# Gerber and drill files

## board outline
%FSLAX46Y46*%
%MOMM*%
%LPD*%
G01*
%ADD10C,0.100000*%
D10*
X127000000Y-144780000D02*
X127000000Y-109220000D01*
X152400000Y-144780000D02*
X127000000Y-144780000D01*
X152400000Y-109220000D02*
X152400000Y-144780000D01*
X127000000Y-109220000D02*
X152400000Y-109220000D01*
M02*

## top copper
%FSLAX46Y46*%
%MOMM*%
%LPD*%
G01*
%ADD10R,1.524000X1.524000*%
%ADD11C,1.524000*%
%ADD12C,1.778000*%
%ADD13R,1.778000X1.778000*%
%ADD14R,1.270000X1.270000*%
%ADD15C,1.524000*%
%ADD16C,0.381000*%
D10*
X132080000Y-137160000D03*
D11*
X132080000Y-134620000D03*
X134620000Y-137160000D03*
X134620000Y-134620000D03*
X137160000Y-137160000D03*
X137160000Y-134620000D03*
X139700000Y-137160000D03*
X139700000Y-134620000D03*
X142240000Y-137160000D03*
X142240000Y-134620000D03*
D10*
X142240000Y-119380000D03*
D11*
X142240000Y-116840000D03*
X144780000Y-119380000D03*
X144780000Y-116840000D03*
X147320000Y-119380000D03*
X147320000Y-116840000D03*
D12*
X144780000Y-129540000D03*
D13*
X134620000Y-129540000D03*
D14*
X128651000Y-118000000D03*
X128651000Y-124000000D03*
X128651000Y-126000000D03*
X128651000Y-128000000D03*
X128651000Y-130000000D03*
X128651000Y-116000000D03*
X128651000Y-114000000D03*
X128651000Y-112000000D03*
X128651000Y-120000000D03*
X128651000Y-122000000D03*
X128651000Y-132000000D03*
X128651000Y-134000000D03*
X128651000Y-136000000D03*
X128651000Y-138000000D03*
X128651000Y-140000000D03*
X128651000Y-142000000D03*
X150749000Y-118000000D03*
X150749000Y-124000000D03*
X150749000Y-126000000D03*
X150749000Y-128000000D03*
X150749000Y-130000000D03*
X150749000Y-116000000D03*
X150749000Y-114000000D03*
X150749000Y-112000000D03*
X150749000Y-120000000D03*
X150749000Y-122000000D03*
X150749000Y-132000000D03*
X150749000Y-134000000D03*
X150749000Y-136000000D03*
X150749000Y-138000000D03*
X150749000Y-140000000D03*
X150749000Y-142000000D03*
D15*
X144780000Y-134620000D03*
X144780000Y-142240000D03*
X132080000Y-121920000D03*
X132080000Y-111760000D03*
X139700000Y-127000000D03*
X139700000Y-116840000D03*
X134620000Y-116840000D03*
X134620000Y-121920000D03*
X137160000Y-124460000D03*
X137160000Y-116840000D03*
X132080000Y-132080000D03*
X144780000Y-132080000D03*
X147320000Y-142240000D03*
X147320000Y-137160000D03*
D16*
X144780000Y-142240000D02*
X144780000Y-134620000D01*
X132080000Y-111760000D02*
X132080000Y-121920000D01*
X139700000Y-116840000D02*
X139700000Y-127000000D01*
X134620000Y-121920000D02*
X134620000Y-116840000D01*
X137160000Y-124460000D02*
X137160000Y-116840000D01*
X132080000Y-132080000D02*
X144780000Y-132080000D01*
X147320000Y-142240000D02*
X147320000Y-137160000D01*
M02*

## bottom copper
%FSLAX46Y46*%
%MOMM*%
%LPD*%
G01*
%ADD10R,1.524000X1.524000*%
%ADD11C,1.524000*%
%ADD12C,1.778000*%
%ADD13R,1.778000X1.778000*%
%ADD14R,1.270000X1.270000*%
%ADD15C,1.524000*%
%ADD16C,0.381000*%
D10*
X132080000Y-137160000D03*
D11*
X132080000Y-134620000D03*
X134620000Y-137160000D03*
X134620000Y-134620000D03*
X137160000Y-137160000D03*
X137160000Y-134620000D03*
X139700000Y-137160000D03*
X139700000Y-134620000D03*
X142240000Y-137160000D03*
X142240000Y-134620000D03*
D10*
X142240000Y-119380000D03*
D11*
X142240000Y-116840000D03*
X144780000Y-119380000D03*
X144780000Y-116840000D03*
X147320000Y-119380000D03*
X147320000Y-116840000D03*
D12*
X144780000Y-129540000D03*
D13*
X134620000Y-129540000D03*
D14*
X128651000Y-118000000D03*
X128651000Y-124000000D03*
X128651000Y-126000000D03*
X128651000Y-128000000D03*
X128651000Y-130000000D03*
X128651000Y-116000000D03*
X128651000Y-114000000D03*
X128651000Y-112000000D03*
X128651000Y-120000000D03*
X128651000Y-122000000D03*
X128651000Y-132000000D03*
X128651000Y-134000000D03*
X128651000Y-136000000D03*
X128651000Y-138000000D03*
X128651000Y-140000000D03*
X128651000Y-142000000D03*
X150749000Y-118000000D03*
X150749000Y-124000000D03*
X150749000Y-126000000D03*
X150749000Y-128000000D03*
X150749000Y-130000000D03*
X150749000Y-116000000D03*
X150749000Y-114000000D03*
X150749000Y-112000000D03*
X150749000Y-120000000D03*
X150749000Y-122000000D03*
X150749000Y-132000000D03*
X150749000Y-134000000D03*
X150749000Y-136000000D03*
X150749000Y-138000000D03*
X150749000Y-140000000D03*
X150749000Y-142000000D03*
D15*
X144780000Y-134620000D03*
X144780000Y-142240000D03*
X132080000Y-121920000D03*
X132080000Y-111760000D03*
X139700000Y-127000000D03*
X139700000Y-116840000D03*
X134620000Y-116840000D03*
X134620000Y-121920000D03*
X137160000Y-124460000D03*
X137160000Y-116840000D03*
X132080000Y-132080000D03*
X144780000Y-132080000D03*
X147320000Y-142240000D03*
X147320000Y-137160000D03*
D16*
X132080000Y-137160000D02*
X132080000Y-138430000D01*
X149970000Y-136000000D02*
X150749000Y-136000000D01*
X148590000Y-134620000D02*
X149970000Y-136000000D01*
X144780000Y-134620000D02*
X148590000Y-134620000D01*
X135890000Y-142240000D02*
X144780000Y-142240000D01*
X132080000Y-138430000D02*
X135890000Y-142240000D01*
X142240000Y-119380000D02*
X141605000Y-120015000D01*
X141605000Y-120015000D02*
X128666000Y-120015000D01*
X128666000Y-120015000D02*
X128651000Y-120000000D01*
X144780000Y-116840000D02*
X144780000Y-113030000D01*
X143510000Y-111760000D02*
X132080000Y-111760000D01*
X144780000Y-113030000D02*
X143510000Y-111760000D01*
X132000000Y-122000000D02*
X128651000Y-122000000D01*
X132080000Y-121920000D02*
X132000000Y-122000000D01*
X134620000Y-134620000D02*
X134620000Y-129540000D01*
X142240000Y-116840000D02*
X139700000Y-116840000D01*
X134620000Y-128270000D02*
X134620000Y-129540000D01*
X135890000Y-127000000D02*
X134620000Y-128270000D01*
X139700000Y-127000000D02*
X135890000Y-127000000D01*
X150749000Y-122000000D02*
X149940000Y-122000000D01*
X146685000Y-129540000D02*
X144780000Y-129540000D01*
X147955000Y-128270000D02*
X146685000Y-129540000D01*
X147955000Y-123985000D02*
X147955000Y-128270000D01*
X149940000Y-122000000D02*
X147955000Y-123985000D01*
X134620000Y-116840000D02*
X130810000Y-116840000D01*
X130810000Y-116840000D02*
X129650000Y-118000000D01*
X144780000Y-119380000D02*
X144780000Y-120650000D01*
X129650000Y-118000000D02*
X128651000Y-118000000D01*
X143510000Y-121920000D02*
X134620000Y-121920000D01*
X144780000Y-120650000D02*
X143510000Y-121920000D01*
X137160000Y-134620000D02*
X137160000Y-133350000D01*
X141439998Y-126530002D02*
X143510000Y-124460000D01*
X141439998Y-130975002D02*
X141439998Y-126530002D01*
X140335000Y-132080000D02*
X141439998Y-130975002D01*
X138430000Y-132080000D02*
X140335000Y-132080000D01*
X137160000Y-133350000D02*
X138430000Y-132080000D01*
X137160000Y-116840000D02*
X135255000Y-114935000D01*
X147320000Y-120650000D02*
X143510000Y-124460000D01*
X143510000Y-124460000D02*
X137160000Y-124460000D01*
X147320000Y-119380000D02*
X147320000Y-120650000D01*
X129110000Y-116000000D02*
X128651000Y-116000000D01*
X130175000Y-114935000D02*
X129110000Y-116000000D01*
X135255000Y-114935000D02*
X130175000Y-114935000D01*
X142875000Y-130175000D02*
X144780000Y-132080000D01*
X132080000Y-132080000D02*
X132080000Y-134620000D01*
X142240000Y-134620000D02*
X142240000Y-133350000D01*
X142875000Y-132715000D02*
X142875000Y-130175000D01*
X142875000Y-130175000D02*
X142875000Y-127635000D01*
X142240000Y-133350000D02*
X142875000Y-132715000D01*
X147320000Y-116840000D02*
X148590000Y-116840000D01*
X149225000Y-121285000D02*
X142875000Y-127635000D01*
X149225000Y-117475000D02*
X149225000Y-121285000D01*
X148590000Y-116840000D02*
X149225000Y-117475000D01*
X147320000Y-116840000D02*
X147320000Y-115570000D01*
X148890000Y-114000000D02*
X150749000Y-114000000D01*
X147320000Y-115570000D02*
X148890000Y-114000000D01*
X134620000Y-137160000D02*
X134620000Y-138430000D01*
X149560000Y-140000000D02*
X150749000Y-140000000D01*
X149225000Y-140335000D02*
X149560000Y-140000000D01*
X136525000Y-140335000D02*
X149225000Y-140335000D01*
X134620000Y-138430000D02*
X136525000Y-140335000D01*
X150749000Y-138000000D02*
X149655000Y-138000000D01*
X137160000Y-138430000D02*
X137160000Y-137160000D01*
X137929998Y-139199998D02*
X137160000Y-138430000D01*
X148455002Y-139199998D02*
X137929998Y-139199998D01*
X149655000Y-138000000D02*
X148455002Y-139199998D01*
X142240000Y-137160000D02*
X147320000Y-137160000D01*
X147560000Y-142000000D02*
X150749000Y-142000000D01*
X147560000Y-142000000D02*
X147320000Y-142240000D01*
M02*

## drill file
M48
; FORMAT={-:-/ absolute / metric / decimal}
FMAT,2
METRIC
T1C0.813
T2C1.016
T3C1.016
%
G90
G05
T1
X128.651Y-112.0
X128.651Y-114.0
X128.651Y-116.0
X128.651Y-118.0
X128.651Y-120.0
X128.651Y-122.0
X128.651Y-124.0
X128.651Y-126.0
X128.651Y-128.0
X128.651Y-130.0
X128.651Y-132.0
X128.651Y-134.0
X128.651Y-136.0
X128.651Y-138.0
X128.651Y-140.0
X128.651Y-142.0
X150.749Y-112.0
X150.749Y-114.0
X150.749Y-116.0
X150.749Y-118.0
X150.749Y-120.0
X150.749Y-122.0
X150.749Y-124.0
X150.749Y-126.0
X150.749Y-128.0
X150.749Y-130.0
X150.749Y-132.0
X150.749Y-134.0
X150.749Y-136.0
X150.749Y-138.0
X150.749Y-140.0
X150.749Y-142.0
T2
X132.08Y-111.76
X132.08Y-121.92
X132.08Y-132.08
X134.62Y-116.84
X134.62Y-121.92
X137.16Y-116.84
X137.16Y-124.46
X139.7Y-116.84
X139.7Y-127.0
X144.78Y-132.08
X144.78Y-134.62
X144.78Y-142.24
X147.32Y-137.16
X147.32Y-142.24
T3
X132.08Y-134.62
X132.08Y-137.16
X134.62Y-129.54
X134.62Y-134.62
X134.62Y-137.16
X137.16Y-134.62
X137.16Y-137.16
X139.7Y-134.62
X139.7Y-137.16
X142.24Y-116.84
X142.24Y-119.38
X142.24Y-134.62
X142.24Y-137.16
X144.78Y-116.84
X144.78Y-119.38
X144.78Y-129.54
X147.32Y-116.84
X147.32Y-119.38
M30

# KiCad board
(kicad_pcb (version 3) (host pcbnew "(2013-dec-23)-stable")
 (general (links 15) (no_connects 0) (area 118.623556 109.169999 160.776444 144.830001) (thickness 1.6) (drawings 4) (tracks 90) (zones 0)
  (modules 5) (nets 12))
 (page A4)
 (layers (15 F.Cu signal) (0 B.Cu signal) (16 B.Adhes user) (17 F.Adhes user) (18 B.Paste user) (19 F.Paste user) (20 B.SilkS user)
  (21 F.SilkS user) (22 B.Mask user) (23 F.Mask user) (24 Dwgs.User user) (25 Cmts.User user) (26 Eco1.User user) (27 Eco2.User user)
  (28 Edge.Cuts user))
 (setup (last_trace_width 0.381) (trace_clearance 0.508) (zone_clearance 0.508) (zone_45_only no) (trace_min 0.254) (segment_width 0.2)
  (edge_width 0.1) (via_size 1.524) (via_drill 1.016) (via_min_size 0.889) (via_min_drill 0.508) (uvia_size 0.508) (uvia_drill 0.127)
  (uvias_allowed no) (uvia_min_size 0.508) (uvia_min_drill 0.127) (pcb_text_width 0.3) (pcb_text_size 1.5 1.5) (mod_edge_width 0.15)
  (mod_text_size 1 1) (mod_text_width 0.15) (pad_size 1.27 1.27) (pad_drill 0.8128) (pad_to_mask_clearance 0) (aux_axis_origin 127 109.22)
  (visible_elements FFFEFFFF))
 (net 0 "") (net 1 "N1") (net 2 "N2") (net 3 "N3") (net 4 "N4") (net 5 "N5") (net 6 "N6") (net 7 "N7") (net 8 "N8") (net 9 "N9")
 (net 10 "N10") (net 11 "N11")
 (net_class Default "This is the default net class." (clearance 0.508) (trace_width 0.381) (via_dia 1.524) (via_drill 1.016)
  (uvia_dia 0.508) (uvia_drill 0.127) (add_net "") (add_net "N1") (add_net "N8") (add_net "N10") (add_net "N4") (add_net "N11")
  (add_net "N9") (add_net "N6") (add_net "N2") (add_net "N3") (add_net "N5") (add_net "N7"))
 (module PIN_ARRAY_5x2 (layer F.Cu) (at 137.16 135.89)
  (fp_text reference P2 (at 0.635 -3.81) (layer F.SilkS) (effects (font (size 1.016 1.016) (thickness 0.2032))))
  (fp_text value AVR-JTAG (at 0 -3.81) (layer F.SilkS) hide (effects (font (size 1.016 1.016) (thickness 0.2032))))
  (pad 1 thru_hole rect (at -5.08 1.27) (size 1.524 1.524) (drill 1.016) (layers *.Cu *.Mask F.SilkS) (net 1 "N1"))
  (pad 2 thru_hole circle (at -5.08 -1.27) (size 1.524 1.524) (drill 1.016) (layers *.Cu *.Mask F.SilkS) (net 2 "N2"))
  (pad 3 thru_hole circle (at -2.54 1.27) (size 1.524 1.524) (drill 1.016) (layers *.Cu *.Mask F.SilkS) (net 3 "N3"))
  (pad 4 thru_hole circle (at -2.54 -1.27) (size 1.524 1.524) (drill 1.016) (layers *.Cu *.Mask F.SilkS) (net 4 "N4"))
  (pad 5 thru_hole circle (at 0 1.27) (size 1.524 1.524) (drill 1.016) (layers *.Cu *.Mask F.SilkS) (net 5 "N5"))
  (pad 6 thru_hole circle (at 0 -1.27) (size 1.524 1.524) (drill 1.016) (layers *.Cu *.Mask F.SilkS) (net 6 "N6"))
  (pad 7 thru_hole circle (at 2.54 1.27) (size 1.524 1.524) (drill 1.016) (layers *.Cu *.Mask F.SilkS))
  (pad 8 thru_hole circle (at 2.54 -1.27) (size 1.524 1.524) (drill 1.016) (layers *.Cu *.Mask F.SilkS))
  (pad 9 thru_hole circle (at 5.08 1.27) (size 1.524 1.524) (drill 1.016) (layers *.Cu *.Mask F.SilkS) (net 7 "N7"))
  (pad 10 thru_hole circle (at 5.08 -1.27) (size 1.524 1.524) (drill 1.016) (layers *.Cu *.Mask F.SilkS) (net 2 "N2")))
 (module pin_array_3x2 (layer F.Cu) (at 144.78 118.11)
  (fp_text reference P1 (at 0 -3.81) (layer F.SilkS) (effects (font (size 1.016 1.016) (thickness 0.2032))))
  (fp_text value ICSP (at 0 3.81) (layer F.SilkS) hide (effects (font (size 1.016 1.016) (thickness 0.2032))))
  (pad 1 thru_hole rect (at -2.54 1.27) (size 1.524 1.524) (drill 1.016) (layers *.Cu *.Mask F.SilkS) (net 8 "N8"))
  (pad 2 thru_hole circle (at -2.54 -1.27) (size 1.524 1.524) (drill 1.016) (layers *.Cu *.Mask F.SilkS) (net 4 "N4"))
  (pad 3 thru_hole circle (at 0 1.27) (size 1.524 1.524) (drill 1.016) (layers *.Cu *.Mask F.SilkS) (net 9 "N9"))
  (pad 4 thru_hole circle (at 0 -1.27) (size 1.524 1.524) (drill 1.016) (layers *.Cu *.Mask F.SilkS) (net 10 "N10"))
  (pad 5 thru_hole circle (at 2.54 1.27) (size 1.524 1.524) (drill 1.016) (layers *.Cu *.Mask F.SilkS) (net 6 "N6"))
  (pad 6 thru_hole circle (at 2.54 -1.27) (size 1.524 1.524) (drill 1.016) (layers *.Cu *.Mask F.SilkS) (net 2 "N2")))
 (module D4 (layer F.Cu) (at 139.7 129.54 180)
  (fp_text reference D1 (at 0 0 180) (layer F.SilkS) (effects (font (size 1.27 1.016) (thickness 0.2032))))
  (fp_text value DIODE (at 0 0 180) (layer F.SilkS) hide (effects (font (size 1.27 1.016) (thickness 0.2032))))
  (pad 1 thru_hole circle (at -5.08 0 180) (size 1.778 1.778) (drill 1.016) (layers *.Cu *.Mask F.SilkS) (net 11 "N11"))
  (pad 2 thru_hole rect (at 5.08 0 180) (size 1.778 1.778) (drill 1.016) (layers *.Cu *.Mask F.SilkS) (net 4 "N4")))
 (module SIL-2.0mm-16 (layer F.Cu) (at 128.651 127)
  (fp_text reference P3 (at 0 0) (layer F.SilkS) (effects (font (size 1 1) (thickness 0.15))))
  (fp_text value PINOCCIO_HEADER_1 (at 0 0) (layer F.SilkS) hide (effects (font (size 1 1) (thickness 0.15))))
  (pad 4 thru_hole rect (at 0 -9) (size 1.27 1.27) (drill 0.8128) (layers *.Cu *.Mask F.SilkS) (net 9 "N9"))
  (pad 7 thru_hole rect (at 0 -3) (size 1.27 1.27) (drill 0.8128) (layers *.Cu *.Mask F.SilkS))
  (pad 8 thru_hole rect (at 0 -1) (size 1.27 1.27) (drill 0.8128) (layers *.Cu *.Mask F.SilkS))
  (pad 9 thru_hole rect (at 0 1) (size 1.27 1.27) (drill 0.8128) (layers *.Cu *.Mask F.SilkS))
  (pad 10 thru_hole rect (at 0 3) (size 1.27 1.27) (drill 0.8128) (layers *.Cu *.Mask F.SilkS))
  (pad 3 thru_hole rect (at 0 -11) (size 1.27 1.27) (drill 0.8128) (layers *.Cu *.Mask F.SilkS) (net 6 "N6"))
  (pad 2 thru_hole rect (at 0 -13) (size 1.27 1.27) (drill 0.8128) (layers *.Cu *.Mask F.SilkS))
  (pad 1 thru_hole rect (at 0 -15) (size 1.27 1.27) (drill 0.8128) (layers *.Cu *.Mask F.SilkS))
  (pad 5 thru_hole rect (at 0 -7) (size 1.27 1.27) (drill 0.8128) (layers *.Cu *.Mask F.SilkS) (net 8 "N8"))
  (pad 6 thru_hole rect (at 0 -5) (size 1.27 1.27) (drill 0.8128) (layers *.Cu *.Mask F.SilkS) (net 10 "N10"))
  (pad 11 thru_hole rect (at 0 5) (size 1.27 1.27) (drill 0.8128) (layers *.Cu *.Mask F.SilkS))
  (pad 12 thru_hole rect (at 0 7) (size 1.27 1.27) (drill 0.8128) (layers *.Cu *.Mask F.SilkS))
  (pad 13 thru_hole rect (at 0 9) (size 1.27 1.27) (drill 0.8128) (layers *.Cu *.Mask F.SilkS))
  (pad 14 thru_hole rect (at 0 11) (size 1.27 1.27) (drill 0.8128) (layers *.Cu *.Mask F.SilkS))
  (pad 15 thru_hole rect (at 0 13) (size 1.27 1.27) (drill 0.8128) (layers *.Cu *.Mask F.SilkS))
  (pad 16 thru_hole rect (at 0 15) (size 1.27 1.27) (drill 0.8128) (layers *.Cu *.Mask F.SilkS)))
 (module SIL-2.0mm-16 (layer F.Cu) (at 150.749 127)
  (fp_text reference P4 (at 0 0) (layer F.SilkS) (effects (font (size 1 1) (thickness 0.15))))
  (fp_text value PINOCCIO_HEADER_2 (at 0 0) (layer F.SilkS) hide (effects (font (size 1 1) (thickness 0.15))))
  (pad 4 thru_hole rect (at 0 -9) (size 1.27 1.27) (drill 0.8128) (layers *.Cu *.Mask F.SilkS))
  (pad 7 thru_hole rect (at 0 -3) (size 1.27 1.27) (drill 0.8128) (layers *.Cu *.Mask F.SilkS))
  (pad 8 thru_hole rect (at 0 -1) (size 1.27 1.27) (drill 0.8128) (layers *.Cu *.Mask F.SilkS))
  (pad 9 thru_hole rect (at 0 1) (size 1.27 1.27) (drill 0.8128) (layers *.Cu *.Mask F.SilkS))
  (pad 10 thru_hole rect (at 0 3) (size 1.27 1.27) (drill 0.8128) (layers *.Cu *.Mask F.SilkS))
  (pad 3 thru_hole rect (at 0 -11) (size 1.27 1.27) (drill 0.8128) (layers *.Cu *.Mask F.SilkS))
  (pad 2 thru_hole rect (at 0 -13) (size 1.27 1.27) (drill 0.8128) (layers *.Cu *.Mask F.SilkS) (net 2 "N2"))
  (pad 1 thru_hole rect (at 0 -15) (size 1.27 1.27) (drill 0.8128) (layers *.Cu *.Mask F.SilkS))
  (pad 5 thru_hole rect (at 0 -7) (size 1.27 1.27) (drill 0.8128) (layers *.Cu *.Mask F.SilkS))
  (pad 6 thru_hole rect (at 0 -5) (size 1.27 1.27) (drill 0.8128) (layers *.Cu *.Mask F.SilkS) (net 11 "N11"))
  (pad 11 thru_hole rect (at 0 5) (size 1.27 1.27) (drill 0.8128) (layers *.Cu *.Mask F.SilkS))
  (pad 12 thru_hole rect (at 0 7) (size 1.27 1.27) (drill 0.8128) (layers *.Cu *.Mask F.SilkS))
  (pad 13 thru_hole rect (at 0 9) (size 1.27 1.27) (drill 0.8128) (layers *.Cu *.Mask F.SilkS) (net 1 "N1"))
  (pad 14 thru_hole rect (at 0 11) (size 1.27 1.27) (drill 0.8128) (layers *.Cu *.Mask F.SilkS) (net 5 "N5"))
  (pad 15 thru_hole rect (at 0 13) (size 1.27 1.27) (drill 0.8128) (layers *.Cu *.Mask F.SilkS) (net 3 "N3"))
  (pad 16 thru_hole rect (at 0 15) (size 1.27 1.27) (drill 0.8128) (layers *.Cu *.Mask F.SilkS) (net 7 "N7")))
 (gr_line (start 127 144.78) (end 127 109.22) (angle 90) (layer Edge.Cuts) (width 0.1))
 (gr_line (start 152.4 144.78) (end 127 144.78) (angle 90) (layer Edge.Cuts) (width 0.1))
 (gr_line (start 152.4 109.22) (end 152.4 144.78) (angle 90) (layer Edge.Cuts) (width 0.1))
 (gr_line (start 127 109.22) (end 152.4 109.22) (angle 90) (layer Edge.Cuts) (width 0.1))
 (segment (start 132.08 137.16) (end 132.08 138.43) (width 0.381) (layer B.Cu) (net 1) (status 10))
 (segment (start 149.97 136) (end 150.749 136) (width 0.381) (layer B.Cu) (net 1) (status 20))
 (segment (start 148.59 134.62) (end 149.97 136) (width 0.381) (layer B.Cu) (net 1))
 (segment (start 144.78 134.62) (end 148.59 134.62) (width 0.381) (layer B.Cu) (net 1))
 (via (at 144.78 134.62) (size 1.524) (layers F.Cu B.Cu) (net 1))
 (segment (start 144.78 142.24) (end 144.78 134.62) (width 0.381) (layer F.Cu) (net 1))
 (via (at 144.78 142.24) (size 1.524) (layers F.Cu B.Cu) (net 1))
 (segment (start 135.89 142.24) (end 144.78 142.24) (width 0.381) (layer B.Cu) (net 1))
 (segment (start 132.08 138.43) (end 135.89 142.24) (width 0.381) (layer B.Cu) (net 1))
 (segment (start 142.24 119.38) (end 141.605 120.015) (width 0.381) (layer B.Cu) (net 8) (status 30))
 (segment (start 141.605 120.015) (end 128.666 120.015) (width 0.381) (layer B.Cu) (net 8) (status 30))
 (segment (start 128.666 120.015) (end 128.651 120) (width 0.381) (layer B.Cu) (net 8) (status 30))
 (segment (start 144.78 116.84) (end 144.78 113.03) (width 0.381) (layer B.Cu) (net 10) (status 10))
 (segment (start 143.51 111.76) (end 132.08 111.76) (width 0.381) (layer B.Cu) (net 10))
 (segment (start 144.78 113.03) (end 143.51 111.76) (width 0.381) (layer B.Cu) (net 10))
 (segment (start 132 122) (end 128.651 122) (width 0.381) (layer B.Cu) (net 10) (status 20))
 (segment (start 132.08 121.92) (end 132 122) (width 0.381) (layer B.Cu) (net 10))
 (via (at 132.08 121.92) (size 1.524) (layers F.Cu B.Cu) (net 10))
 (segment (start 132.08 111.76) (end 132.08 121.92) (width 0.381) (layer F.Cu) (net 10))
 (via (at 132.08 111.76) (size 1.524) (layers F.Cu B.Cu) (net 10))
 (segment (start 134.62 134.62) (end 134.62 129.54) (width 0.381) (layer B.Cu) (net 4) (status 30))
 (segment (start 142.24 116.84) (end 139.7 116.84) (width 0.381) (layer B.Cu) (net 4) (status 10))
 (segment (start 134.62 128.27) (end 134.62 129.54) (width 0.381) (layer B.Cu) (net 4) (status 20))
 (segment (start 135.89 127) (end 134.62 128.27) (width 0.381) (layer B.Cu) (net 4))
 (segment (start 139.7 127) (end 135.89 127) (width 0.381) (layer B.Cu) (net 4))
 (via (at 139.7 127) (size 1.524) (layers F.Cu B.Cu) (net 4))
 (segment (start 139.7 116.84) (end 139.7 127) (width 0.381) (layer F.Cu) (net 4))
 (via (at 139.7 116.84) (size 1.524) (layers F.Cu B.Cu) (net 4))
 (segment (start 150.749 122) (end 149.94 122) (width 0.381) (layer B.Cu) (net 11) (status 10))
 (segment (start 146.685 129.54) (end 144.78 129.54) (width 0.381) (layer B.Cu) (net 11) (status 20))
 (segment (start 147.955 128.27) (end 146.685 129.54) (width 0.381) (layer B.Cu) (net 11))
 (segment (start 147.955 123.985) (end 147.955 128.27) (width 0.381) (layer B.Cu) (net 11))
 (segment (start 149.94 122) (end 147.955 123.985) (width 0.381) (layer B.Cu) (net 11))
 (segment (start 134.62 116.84) (end 130.81 116.84) (width 0.381) (layer B.Cu) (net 9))
 (segment (start 130.81 116.84) (end 129.65 118) (width 0.381) (layer B.Cu) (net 9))
 (segment (start 144.78 119.38) (end 144.78 120.65) (width 0.381) (layer B.Cu) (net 9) (status 10))
 (segment (start 129.65 118) (end 128.651 118) (width 0.381) (layer B.Cu) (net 9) (status 20))
 (via (at 134.62 116.84) (size 1.524) (layers F.Cu B.Cu) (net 9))
 (segment (start 134.62 121.92) (end 134.62 116.84) (width 0.381) (layer F.Cu) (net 9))
 (via (at 134.62 121.92) (size 1.524) (layers F.Cu B.Cu) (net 9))
 (segment (start 143.51 121.92) (end 134.62 121.92) (width 0.381) (layer B.Cu) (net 9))
 (segment (start 144.78 120.65) (end 143.51 121.92) (width 0.381) (layer B.Cu) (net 9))
 (segment (start 137.16 134.62) (end 137.16 133.35) (width 0.381) (layer B.Cu) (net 6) (status 10))
 (segment (start 141.439998 126.530002) (end 143.51 124.46) (width 0.381) (layer B.Cu) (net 6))
 (segment (start 141.439998 130.975002) (end 141.439998 126.530002) (width 0.381) (layer B.Cu) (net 6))
 (segment (start 140.335 132.08) (end 141.439998 130.975002) (width 0.381) (layer B.Cu) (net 6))
 (segment (start 138.43 132.08) (end 140.335 132.08) (width 0.381) (layer B.Cu) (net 6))
 (segment (start 137.16 133.35) (end 138.43 132.08) (width 0.381) (layer B.Cu) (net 6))
 (segment (start 137.16 116.84) (end 135.255 114.935) (width 0.381) (layer B.Cu) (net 6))
 (segment (start 147.32 120.65) (end 143.51 124.46) (width 0.381) (layer B.Cu) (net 6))
 (segment (start 143.51 124.46) (end 137.16 124.46) (width 0.381) (layer B.Cu) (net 6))
 (via (at 137.16 124.46) (size 1.524) (layers F.Cu B.Cu) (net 6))
 (segment (start 137.16 124.46) (end 137.16 116.84) (width 0.381) (layer F.Cu) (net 6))
 (via (at 137.16 116.84) (size 1.524) (layers F.Cu B.Cu) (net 6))
 (segment (start 147.32 119.38) (end 147.32 120.65) (width 0.381) (layer B.Cu) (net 6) (status 10))
 (segment (start 129.11 116) (end 128.651 116) (width 0.381) (layer B.Cu) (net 6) (status 30))
 (segment (start 130.175 114.935) (end 129.11 116) (width 0.381) (layer B.Cu) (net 6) (status 20))
 (segment (start 135.255 114.935) (end 130.175 114.935) (width 0.381) (layer B.Cu) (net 6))
 (segment (start 142.875 130.175) (end 144.78 132.08) (width 0.381) (layer B.Cu) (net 2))
 (via (at 132.08 132.08) (size 1.524) (layers F.Cu B.Cu) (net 2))
 (segment (start 132.08 132.08) (end 144.78 132.08) (width 0.381) (layer F.Cu) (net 2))
 (via (at 144.78 132.08) (size 1.524) (layers F.Cu B.Cu) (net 2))
 (segment (start 132.08 132.08) (end 132.08 134.62) (width 0.381) (layer B.Cu) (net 2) (status 10))
 (segment (start 142.24 134.62) (end 142.24 133.35) (width 0.381) (layer B.Cu) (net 2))
 (segment (start 142.875 132.715) (end 142.875 130.175) (width 0.381) (layer B.Cu) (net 2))
 (segment (start 142.875 130.175) (end 142.875 127.635) (width 0.381) (layer B.Cu) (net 2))
 (segment (start 142.24 133.35) (end 142.875 132.715) (width 0.381) (layer B.Cu) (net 2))
 (segment (start 147.32 116.84) (end 148.59 116.84) (width 0.381) (layer B.Cu) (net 2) (status 10))
 (segment (start 149.225 121.285) (end 142.875 127.635) (width 0.381) (layer B.Cu) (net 2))
 (segment (start 149.225 117.475) (end 149.225 121.285) (width 0.381) (layer B.Cu) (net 2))
 (segment (start 148.59 116.84) (end 149.225 117.475) (width 0.381) (layer B.Cu) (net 2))
 (segment (start 147.32 116.84) (end 147.32 115.57) (width 0.381) (layer B.Cu) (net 2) (status 10))
 (segment (start 148.89 114) (end 150.749 114) (width 0.381) (layer B.Cu) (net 2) (status 20))
 (segment (start 147.32 115.57) (end 148.89 114) (width 0.381) (layer B.Cu) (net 2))
 (segment (start 134.62 137.16) (end 134.62 138.43) (width 0.381) (layer B.Cu) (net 3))
 (segment (start 149.56 140) (end 150.749 140) (width 0.381) (layer B.Cu) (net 3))
 (segment (start 149.225 140.335) (end 149.56 140) (width 0.381) (layer B.Cu) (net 3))
 (segment (start 136.525 140.335) (end 149.225 140.335) (width 0.381) (layer B.Cu) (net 3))
 (segment (start 134.62 138.43) (end 136.525 140.335) (width 0.381) (layer B.Cu) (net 3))
 (segment (start 150.749 138) (end 149.655 138) (width 0.381) (layer B.Cu) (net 5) (status 10))
 (segment (start 137.16 138.43) (end 137.16 137.16) (width 0.381) (layer B.Cu) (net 5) (status 20))
 (segment (start 137.929998 139.199998) (end 137.16 138.43) (width 0.381) (layer B.Cu) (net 5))
 (segment (start 148.455002 139.199998) (end 137.929998 139.199998) (width 0.381) (layer B.Cu) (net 5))
 (segment (start 149.655 138) (end 148.455002 139.199998) (width 0.381) (layer B.Cu) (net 5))
 (segment (start 142.24 137.16) (end 147.32 137.16) (width 0.381) (layer B.Cu) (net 7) (status 10))
 (segment (start 147.56 142) (end 150.749 142) (width 0.381) (layer B.Cu) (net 7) (status 20))
 (segment (start 147.32 142.24) (end 147.32 137.16) (width 0.381) (layer F.Cu) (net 7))
 (via (at 147.32 142.24) (size 1.524) (layers F.Cu B.Cu) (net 7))
 (segment (start 147.56 142) (end 147.32 142.24) (width 0.381) (layer B.Cu) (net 7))
 (via (at 147.32 137.16) (size 1.524) (layers F.Cu B.Cu) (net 7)))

